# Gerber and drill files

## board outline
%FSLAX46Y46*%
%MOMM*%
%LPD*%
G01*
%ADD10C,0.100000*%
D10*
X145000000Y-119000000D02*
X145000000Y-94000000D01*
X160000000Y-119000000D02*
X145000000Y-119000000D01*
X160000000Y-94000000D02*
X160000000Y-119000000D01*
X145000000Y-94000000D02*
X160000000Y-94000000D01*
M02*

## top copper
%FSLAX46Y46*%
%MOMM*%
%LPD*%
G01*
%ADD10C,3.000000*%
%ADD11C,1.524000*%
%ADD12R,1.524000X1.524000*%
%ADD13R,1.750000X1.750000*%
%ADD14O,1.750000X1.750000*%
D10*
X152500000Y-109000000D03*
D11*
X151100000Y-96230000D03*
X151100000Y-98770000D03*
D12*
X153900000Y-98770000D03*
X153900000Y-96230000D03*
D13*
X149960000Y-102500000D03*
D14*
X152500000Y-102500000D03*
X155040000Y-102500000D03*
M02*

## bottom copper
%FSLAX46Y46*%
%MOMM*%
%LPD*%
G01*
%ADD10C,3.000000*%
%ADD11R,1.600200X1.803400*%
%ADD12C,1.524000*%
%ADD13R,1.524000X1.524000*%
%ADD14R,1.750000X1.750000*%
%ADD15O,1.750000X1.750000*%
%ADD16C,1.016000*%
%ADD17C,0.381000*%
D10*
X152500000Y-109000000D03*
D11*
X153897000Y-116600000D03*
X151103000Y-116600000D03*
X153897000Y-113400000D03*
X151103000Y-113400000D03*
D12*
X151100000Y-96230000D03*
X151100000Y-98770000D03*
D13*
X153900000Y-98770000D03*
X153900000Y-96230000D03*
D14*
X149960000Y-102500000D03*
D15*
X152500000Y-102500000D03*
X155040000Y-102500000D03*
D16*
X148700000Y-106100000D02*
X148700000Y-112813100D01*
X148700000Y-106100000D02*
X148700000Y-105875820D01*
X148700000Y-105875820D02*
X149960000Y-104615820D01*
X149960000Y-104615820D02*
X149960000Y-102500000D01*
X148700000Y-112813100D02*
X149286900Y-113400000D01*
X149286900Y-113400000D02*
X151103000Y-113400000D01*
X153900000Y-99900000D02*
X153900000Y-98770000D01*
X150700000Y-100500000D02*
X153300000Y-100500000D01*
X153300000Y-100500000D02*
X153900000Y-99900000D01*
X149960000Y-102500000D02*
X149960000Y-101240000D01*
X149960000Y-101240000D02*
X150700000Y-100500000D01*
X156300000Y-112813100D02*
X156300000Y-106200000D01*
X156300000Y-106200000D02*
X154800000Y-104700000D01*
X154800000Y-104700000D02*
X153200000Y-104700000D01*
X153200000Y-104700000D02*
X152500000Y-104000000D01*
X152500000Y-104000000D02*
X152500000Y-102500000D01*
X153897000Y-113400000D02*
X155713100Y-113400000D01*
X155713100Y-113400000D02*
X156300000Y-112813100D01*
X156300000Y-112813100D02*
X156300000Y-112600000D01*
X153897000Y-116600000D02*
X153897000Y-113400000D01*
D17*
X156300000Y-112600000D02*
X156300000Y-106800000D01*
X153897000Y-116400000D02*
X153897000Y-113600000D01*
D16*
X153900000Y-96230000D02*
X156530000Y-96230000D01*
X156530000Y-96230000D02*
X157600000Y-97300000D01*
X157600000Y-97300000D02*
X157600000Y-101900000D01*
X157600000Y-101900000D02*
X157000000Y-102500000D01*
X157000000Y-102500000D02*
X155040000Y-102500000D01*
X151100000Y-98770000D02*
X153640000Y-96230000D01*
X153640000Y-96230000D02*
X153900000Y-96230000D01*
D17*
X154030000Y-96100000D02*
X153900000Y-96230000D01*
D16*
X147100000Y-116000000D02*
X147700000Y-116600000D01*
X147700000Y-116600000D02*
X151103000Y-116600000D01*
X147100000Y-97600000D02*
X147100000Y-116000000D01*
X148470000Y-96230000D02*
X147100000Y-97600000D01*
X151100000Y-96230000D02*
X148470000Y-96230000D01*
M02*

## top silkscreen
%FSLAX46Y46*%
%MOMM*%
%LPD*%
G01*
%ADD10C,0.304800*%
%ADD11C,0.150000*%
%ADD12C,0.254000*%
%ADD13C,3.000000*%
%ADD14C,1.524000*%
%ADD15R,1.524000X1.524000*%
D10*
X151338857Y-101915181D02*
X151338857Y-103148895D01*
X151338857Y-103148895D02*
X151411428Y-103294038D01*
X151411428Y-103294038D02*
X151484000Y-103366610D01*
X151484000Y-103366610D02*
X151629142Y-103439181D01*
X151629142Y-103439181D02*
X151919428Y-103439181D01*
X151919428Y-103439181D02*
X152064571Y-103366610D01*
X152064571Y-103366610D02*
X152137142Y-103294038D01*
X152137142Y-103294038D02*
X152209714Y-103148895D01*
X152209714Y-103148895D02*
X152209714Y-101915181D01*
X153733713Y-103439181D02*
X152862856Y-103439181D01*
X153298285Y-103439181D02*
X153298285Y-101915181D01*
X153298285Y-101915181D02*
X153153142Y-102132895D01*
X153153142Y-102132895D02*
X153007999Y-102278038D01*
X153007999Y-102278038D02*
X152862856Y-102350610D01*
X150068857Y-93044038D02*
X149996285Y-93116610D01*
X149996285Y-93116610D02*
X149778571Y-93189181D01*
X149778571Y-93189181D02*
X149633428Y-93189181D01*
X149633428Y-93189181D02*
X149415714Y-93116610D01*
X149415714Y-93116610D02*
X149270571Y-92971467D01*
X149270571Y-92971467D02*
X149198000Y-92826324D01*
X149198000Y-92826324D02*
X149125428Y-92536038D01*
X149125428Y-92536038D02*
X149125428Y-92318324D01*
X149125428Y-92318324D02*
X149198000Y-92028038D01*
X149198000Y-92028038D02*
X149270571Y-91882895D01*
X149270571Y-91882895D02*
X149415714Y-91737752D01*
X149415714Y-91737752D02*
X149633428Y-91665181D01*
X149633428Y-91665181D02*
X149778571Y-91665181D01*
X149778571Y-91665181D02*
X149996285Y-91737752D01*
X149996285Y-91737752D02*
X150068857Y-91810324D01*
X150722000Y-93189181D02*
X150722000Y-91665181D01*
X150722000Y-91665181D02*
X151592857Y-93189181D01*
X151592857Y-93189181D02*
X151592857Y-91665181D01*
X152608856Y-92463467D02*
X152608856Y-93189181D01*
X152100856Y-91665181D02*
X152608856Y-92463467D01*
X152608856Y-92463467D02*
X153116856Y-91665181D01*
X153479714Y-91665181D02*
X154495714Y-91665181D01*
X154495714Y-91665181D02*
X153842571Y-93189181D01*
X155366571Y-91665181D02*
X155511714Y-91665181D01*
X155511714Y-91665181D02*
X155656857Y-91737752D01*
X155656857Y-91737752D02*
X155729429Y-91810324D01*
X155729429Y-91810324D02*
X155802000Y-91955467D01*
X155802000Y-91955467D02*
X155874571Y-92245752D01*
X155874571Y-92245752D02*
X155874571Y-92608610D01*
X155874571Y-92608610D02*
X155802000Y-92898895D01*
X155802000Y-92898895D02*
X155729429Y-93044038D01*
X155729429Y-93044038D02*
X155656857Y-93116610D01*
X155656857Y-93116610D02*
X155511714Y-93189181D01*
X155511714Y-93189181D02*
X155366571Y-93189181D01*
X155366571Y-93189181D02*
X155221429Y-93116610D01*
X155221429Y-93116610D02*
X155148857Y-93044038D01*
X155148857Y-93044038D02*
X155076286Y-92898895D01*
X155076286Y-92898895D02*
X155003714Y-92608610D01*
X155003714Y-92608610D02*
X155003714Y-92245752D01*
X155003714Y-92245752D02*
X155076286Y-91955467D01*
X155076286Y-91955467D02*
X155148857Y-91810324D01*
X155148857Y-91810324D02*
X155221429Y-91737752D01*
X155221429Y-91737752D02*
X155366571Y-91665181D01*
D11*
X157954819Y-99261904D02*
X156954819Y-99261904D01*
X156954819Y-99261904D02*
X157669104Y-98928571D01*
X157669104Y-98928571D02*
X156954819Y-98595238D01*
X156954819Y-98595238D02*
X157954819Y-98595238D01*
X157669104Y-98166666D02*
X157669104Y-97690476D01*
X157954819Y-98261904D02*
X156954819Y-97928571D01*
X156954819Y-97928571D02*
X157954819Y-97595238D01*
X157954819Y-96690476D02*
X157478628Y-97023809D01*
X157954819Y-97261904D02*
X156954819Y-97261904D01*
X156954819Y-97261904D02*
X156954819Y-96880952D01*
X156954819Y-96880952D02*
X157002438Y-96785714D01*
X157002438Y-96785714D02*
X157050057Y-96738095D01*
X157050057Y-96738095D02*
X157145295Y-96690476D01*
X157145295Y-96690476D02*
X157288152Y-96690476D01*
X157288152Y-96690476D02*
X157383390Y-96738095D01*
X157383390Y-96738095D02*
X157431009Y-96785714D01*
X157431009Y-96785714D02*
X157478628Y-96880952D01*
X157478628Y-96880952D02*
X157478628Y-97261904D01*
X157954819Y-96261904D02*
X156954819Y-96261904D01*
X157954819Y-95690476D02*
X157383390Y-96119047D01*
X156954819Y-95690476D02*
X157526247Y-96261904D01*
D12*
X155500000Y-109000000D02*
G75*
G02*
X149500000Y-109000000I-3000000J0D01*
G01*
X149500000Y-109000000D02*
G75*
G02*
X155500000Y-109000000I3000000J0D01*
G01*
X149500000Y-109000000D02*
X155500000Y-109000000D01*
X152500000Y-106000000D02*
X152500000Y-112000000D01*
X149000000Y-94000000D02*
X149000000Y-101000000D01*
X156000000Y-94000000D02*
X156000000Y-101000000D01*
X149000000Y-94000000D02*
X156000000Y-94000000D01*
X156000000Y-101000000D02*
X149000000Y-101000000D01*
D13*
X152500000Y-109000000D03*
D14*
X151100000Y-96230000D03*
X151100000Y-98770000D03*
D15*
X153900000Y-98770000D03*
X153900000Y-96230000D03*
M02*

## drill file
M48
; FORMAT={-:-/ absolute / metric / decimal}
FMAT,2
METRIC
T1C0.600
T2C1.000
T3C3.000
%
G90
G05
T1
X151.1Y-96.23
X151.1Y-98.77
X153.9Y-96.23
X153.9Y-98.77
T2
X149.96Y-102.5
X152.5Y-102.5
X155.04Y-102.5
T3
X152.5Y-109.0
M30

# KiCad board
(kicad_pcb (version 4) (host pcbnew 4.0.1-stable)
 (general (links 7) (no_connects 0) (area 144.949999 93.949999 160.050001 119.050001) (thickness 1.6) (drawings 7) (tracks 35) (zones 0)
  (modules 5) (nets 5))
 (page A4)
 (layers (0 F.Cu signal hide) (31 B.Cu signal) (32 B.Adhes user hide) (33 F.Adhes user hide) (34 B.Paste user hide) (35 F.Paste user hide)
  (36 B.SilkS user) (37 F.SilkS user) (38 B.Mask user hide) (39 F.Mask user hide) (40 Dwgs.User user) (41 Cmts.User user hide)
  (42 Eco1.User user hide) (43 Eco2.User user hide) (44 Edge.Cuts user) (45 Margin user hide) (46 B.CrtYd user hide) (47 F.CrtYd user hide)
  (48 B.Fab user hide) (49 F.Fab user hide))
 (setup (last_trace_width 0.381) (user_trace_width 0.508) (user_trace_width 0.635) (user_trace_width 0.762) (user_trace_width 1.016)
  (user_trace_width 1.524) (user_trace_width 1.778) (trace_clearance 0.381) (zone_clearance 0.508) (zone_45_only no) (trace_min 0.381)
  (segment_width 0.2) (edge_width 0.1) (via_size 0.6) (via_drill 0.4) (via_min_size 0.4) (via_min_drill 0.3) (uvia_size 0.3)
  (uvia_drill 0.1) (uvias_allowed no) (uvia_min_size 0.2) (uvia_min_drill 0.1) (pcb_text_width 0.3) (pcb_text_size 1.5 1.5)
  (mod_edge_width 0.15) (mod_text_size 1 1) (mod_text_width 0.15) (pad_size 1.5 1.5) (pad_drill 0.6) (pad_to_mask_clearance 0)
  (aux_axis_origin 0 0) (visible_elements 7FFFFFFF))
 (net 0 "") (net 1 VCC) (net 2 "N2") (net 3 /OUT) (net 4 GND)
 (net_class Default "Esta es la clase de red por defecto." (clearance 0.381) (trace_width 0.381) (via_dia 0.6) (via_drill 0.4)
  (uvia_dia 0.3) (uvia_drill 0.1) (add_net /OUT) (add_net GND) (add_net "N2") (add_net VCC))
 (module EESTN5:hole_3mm (layer F.Cu) (at 152.5 109)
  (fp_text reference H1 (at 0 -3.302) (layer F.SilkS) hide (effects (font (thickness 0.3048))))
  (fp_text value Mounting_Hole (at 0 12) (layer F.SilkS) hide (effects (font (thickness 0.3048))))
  (fp_circle (center 0 0) (end 3 0) (layer F.SilkS) (width 0.254))
  (fp_line (start -3 0) (end 3 0) (layer F.SilkS) (width 0.254))
  (fp_line (start 0 -3) (end 0 3) (layer F.SilkS) (width 0.254))
  (pad 1 thru_hole circle (at 0 0) (size 3 3) (drill 3) (layers *.Cu F.SilkS)))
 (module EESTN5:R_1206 (layer B.Cu) (at 152.5 116.6)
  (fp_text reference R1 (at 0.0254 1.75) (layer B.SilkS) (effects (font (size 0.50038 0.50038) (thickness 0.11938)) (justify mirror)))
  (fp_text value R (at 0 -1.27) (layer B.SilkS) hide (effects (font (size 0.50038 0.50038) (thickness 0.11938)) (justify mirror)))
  (pad 1 smd rect (at 1.397 0) (size 1.6002 1.8034) (layers B.Cu B.Paste B.Mask) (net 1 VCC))
  (pad 2 smd rect (at -1.397 0) (size 1.6002 1.8034) (layers B.Cu B.Paste B.Mask) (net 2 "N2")))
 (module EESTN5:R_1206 (layer B.Cu) (at 152.5 113.4)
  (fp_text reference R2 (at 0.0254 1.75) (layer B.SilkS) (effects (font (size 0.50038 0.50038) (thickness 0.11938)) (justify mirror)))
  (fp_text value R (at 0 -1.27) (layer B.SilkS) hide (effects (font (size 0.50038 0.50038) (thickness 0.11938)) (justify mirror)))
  (pad 1 smd rect (at 1.397 0) (size 1.6002 1.8034) (layers B.Cu B.Paste B.Mask) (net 1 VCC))
  (pad 2 smd rect (at -1.397 0) (size 1.6002 1.8034) (layers B.Cu B.Paste B.Mask) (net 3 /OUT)))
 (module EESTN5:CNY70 (layer F.Cu) (at 152.5 97.5)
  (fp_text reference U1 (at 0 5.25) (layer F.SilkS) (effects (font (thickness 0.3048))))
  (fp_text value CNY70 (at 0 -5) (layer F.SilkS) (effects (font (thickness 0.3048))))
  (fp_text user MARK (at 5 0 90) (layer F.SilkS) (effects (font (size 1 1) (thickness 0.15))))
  (fp_line (start -3.5 -3.5) (end -3.5 3.5) (layer F.SilkS) (width 0.254))
  (fp_line (start 3.5 -3.5) (end 3.5 3.5) (layer F.SilkS) (width 0.254))
  (fp_line (start -3.5 -3.5) (end 3.5 -3.5) (layer F.SilkS) (width 0.254))
  (fp_line (start 3.5 3.5) (end -3.5 3.5) (layer F.SilkS) (width 0.254))
  (pad 1 thru_hole circle (at -1.4 -1.27) (size 1.524 1.524) (drill 0.6) (layers *.Cu *.Mask F.SilkS) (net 2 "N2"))
  (pad 2 thru_hole circle (at -1.4 1.27) (size 1.524 1.524) (drill 0.6) (layers *.Cu *.Mask F.SilkS) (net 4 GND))
  (pad 3 thru_hole rect (at 1.4 1.27) (size 1.524 1.524) (drill 0.6) (layers *.Cu *.Mask F.SilkS) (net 3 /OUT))
  (pad 4 thru_hole rect (at 1.4 -1.27) (size 1.524 1.524) (drill 0.6) (layers *.Cu *.Mask F.SilkS) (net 4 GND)))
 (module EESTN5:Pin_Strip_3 (layer B.Cu) (at 152.5 102.5)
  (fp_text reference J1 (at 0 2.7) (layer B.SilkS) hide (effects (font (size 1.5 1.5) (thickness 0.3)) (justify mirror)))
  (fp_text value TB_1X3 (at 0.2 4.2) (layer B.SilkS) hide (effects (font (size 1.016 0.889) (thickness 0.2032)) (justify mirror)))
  (pad 1 thru_hole rect (at -2.54 0) (size 1.75 1.75) (drill 1) (layers *.Cu *.Mask B.SilkS) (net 3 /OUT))
  (pad 2 thru_hole oval (at 0 0) (size 1.75 1.75) (drill 1) (layers *.Cu *.Mask B.SilkS) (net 1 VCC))
  (pad 3 thru_hole oval (at 2.54 0) (size 1.75 1.75) (drill 1) (layers *.Cu *.Mask B.SilkS) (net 4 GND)))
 (gr_line (start 145 119) (end 145 94) (angle 90) (layer Edge.Cuts) (width 0.1))
 (gr_line (start 160 119) (end 145 119) (angle 90) (layer Edge.Cuts) (width 0.1))
 (gr_line (start 160 94) (end 160 119) (angle 90) (layer Edge.Cuts) (width 0.1))
 (gr_line (start 145 94) (end 160 94) (angle 90) (layer Edge.Cuts) (width 0.1))
 (segment (start 148.7 106.1) (end 148.7 112.8131) (width 1.016) (layer B.Cu) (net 3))
 (segment (start 148.7 106.1) (end 148.7 105.87582) (width 1.016) (layer B.Cu) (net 3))
 (segment (start 148.7 105.87582) (end 149.96 104.61582) (width 1.016) (layer B.Cu) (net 3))
 (segment (start 149.96 104.61582) (end 149.96 102.5) (width 1.016) (layer B.Cu) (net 3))
 (segment (start 148.7 112.8131) (end 149.2869 113.4) (width 1.016) (layer B.Cu) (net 3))
 (segment (start 149.2869 113.4) (end 151.103 113.4) (width 1.016) (layer B.Cu) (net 3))
 (segment (start 153.9 99.9) (end 153.9 98.77) (width 1.016) (layer B.Cu) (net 3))
 (segment (start 150.7 100.5) (end 153.3 100.5) (width 1.016) (layer B.Cu) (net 3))
 (segment (start 153.3 100.5) (end 153.9 99.9) (width 1.016) (layer B.Cu) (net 3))
 (segment (start 149.96 102.5) (end 149.96 101.24) (width 1.016) (layer B.Cu) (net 3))
 (segment (start 149.96 101.24) (end 150.7 100.5) (width 1.016) (layer B.Cu) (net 3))
 (segment (start 156.3 112.8131) (end 156.3 106.2) (width 1.016) (layer B.Cu) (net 1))
 (segment (start 156.3 106.2) (end 154.8 104.7) (width 1.016) (layer B.Cu) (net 1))
 (segment (start 154.8 104.7) (end 153.2 104.7) (width 1.016) (layer B.Cu) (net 1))
 (segment (start 153.2 104.7) (end 152.5 104) (width 1.016) (layer B.Cu) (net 1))
 (segment (start 152.5 104) (end 152.5 102.5) (width 1.016) (layer B.Cu) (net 1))
 (segment (start 153.897 113.4) (end 155.7131 113.4) (width 1.016) (layer B.Cu) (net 1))
 (segment (start 155.7131 113.4) (end 156.3 112.8131) (width 1.016) (layer B.Cu) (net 1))
 (segment (start 156.3 112.8131) (end 156.3 112.6) (width 1.016) (layer B.Cu) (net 1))
 (segment (start 153.897 116.6) (end 153.897 113.4) (width 1.016) (layer B.Cu) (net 1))
 (segment (start 156.3 112.6) (end 156.3 106.8) (width 0.381) (layer B.Cu) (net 1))
 (segment (start 153.897 116.4) (end 153.897 113.6) (width 0.381) (layer B.Cu) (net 1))
 (segment (start 153.9 96.23) (end 156.53 96.23) (width 1.016) (layer B.Cu) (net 4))
 (segment (start 156.53 96.23) (end 157.6 97.3) (width 1.016) (layer B.Cu) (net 4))
 (segment (start 157.6 97.3) (end 157.6 101.9) (width 1.016) (layer B.Cu) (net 4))
 (segment (start 157.6 101.9) (end 157 102.5) (width 1.016) (layer B.Cu) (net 4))
 (segment (start 157 102.5) (end 155.04 102.5) (width 1.016) (layer B.Cu) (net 4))
 (segment (start 151.1 98.77) (end 153.64 96.23) (width 1.016) (layer B.Cu) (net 4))
 (segment (start 153.64 96.23) (end 153.9 96.23) (width 1.016) (layer B.Cu) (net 4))
 (segment (start 154.03 96.1) (end 153.9 96.23) (width 0.381) (layer B.Cu) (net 4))
 (segment (start 147.1 116) (end 147.7 116.6) (width 1.016) (layer B.Cu) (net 2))
 (segment (start 147.7 116.6) (end 151.103 116.6) (width 1.016) (layer B.Cu) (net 2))
 (segment (start 147.1 97.6) (end 147.1 116) (width 1.016) (layer B.Cu) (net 2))
 (segment (start 148.47 96.23) (end 147.1 97.6) (width 1.016) (layer B.Cu) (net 2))
 (segment (start 151.1 96.23) (end 148.47 96.23) (width 1.016) (layer B.Cu) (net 2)))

